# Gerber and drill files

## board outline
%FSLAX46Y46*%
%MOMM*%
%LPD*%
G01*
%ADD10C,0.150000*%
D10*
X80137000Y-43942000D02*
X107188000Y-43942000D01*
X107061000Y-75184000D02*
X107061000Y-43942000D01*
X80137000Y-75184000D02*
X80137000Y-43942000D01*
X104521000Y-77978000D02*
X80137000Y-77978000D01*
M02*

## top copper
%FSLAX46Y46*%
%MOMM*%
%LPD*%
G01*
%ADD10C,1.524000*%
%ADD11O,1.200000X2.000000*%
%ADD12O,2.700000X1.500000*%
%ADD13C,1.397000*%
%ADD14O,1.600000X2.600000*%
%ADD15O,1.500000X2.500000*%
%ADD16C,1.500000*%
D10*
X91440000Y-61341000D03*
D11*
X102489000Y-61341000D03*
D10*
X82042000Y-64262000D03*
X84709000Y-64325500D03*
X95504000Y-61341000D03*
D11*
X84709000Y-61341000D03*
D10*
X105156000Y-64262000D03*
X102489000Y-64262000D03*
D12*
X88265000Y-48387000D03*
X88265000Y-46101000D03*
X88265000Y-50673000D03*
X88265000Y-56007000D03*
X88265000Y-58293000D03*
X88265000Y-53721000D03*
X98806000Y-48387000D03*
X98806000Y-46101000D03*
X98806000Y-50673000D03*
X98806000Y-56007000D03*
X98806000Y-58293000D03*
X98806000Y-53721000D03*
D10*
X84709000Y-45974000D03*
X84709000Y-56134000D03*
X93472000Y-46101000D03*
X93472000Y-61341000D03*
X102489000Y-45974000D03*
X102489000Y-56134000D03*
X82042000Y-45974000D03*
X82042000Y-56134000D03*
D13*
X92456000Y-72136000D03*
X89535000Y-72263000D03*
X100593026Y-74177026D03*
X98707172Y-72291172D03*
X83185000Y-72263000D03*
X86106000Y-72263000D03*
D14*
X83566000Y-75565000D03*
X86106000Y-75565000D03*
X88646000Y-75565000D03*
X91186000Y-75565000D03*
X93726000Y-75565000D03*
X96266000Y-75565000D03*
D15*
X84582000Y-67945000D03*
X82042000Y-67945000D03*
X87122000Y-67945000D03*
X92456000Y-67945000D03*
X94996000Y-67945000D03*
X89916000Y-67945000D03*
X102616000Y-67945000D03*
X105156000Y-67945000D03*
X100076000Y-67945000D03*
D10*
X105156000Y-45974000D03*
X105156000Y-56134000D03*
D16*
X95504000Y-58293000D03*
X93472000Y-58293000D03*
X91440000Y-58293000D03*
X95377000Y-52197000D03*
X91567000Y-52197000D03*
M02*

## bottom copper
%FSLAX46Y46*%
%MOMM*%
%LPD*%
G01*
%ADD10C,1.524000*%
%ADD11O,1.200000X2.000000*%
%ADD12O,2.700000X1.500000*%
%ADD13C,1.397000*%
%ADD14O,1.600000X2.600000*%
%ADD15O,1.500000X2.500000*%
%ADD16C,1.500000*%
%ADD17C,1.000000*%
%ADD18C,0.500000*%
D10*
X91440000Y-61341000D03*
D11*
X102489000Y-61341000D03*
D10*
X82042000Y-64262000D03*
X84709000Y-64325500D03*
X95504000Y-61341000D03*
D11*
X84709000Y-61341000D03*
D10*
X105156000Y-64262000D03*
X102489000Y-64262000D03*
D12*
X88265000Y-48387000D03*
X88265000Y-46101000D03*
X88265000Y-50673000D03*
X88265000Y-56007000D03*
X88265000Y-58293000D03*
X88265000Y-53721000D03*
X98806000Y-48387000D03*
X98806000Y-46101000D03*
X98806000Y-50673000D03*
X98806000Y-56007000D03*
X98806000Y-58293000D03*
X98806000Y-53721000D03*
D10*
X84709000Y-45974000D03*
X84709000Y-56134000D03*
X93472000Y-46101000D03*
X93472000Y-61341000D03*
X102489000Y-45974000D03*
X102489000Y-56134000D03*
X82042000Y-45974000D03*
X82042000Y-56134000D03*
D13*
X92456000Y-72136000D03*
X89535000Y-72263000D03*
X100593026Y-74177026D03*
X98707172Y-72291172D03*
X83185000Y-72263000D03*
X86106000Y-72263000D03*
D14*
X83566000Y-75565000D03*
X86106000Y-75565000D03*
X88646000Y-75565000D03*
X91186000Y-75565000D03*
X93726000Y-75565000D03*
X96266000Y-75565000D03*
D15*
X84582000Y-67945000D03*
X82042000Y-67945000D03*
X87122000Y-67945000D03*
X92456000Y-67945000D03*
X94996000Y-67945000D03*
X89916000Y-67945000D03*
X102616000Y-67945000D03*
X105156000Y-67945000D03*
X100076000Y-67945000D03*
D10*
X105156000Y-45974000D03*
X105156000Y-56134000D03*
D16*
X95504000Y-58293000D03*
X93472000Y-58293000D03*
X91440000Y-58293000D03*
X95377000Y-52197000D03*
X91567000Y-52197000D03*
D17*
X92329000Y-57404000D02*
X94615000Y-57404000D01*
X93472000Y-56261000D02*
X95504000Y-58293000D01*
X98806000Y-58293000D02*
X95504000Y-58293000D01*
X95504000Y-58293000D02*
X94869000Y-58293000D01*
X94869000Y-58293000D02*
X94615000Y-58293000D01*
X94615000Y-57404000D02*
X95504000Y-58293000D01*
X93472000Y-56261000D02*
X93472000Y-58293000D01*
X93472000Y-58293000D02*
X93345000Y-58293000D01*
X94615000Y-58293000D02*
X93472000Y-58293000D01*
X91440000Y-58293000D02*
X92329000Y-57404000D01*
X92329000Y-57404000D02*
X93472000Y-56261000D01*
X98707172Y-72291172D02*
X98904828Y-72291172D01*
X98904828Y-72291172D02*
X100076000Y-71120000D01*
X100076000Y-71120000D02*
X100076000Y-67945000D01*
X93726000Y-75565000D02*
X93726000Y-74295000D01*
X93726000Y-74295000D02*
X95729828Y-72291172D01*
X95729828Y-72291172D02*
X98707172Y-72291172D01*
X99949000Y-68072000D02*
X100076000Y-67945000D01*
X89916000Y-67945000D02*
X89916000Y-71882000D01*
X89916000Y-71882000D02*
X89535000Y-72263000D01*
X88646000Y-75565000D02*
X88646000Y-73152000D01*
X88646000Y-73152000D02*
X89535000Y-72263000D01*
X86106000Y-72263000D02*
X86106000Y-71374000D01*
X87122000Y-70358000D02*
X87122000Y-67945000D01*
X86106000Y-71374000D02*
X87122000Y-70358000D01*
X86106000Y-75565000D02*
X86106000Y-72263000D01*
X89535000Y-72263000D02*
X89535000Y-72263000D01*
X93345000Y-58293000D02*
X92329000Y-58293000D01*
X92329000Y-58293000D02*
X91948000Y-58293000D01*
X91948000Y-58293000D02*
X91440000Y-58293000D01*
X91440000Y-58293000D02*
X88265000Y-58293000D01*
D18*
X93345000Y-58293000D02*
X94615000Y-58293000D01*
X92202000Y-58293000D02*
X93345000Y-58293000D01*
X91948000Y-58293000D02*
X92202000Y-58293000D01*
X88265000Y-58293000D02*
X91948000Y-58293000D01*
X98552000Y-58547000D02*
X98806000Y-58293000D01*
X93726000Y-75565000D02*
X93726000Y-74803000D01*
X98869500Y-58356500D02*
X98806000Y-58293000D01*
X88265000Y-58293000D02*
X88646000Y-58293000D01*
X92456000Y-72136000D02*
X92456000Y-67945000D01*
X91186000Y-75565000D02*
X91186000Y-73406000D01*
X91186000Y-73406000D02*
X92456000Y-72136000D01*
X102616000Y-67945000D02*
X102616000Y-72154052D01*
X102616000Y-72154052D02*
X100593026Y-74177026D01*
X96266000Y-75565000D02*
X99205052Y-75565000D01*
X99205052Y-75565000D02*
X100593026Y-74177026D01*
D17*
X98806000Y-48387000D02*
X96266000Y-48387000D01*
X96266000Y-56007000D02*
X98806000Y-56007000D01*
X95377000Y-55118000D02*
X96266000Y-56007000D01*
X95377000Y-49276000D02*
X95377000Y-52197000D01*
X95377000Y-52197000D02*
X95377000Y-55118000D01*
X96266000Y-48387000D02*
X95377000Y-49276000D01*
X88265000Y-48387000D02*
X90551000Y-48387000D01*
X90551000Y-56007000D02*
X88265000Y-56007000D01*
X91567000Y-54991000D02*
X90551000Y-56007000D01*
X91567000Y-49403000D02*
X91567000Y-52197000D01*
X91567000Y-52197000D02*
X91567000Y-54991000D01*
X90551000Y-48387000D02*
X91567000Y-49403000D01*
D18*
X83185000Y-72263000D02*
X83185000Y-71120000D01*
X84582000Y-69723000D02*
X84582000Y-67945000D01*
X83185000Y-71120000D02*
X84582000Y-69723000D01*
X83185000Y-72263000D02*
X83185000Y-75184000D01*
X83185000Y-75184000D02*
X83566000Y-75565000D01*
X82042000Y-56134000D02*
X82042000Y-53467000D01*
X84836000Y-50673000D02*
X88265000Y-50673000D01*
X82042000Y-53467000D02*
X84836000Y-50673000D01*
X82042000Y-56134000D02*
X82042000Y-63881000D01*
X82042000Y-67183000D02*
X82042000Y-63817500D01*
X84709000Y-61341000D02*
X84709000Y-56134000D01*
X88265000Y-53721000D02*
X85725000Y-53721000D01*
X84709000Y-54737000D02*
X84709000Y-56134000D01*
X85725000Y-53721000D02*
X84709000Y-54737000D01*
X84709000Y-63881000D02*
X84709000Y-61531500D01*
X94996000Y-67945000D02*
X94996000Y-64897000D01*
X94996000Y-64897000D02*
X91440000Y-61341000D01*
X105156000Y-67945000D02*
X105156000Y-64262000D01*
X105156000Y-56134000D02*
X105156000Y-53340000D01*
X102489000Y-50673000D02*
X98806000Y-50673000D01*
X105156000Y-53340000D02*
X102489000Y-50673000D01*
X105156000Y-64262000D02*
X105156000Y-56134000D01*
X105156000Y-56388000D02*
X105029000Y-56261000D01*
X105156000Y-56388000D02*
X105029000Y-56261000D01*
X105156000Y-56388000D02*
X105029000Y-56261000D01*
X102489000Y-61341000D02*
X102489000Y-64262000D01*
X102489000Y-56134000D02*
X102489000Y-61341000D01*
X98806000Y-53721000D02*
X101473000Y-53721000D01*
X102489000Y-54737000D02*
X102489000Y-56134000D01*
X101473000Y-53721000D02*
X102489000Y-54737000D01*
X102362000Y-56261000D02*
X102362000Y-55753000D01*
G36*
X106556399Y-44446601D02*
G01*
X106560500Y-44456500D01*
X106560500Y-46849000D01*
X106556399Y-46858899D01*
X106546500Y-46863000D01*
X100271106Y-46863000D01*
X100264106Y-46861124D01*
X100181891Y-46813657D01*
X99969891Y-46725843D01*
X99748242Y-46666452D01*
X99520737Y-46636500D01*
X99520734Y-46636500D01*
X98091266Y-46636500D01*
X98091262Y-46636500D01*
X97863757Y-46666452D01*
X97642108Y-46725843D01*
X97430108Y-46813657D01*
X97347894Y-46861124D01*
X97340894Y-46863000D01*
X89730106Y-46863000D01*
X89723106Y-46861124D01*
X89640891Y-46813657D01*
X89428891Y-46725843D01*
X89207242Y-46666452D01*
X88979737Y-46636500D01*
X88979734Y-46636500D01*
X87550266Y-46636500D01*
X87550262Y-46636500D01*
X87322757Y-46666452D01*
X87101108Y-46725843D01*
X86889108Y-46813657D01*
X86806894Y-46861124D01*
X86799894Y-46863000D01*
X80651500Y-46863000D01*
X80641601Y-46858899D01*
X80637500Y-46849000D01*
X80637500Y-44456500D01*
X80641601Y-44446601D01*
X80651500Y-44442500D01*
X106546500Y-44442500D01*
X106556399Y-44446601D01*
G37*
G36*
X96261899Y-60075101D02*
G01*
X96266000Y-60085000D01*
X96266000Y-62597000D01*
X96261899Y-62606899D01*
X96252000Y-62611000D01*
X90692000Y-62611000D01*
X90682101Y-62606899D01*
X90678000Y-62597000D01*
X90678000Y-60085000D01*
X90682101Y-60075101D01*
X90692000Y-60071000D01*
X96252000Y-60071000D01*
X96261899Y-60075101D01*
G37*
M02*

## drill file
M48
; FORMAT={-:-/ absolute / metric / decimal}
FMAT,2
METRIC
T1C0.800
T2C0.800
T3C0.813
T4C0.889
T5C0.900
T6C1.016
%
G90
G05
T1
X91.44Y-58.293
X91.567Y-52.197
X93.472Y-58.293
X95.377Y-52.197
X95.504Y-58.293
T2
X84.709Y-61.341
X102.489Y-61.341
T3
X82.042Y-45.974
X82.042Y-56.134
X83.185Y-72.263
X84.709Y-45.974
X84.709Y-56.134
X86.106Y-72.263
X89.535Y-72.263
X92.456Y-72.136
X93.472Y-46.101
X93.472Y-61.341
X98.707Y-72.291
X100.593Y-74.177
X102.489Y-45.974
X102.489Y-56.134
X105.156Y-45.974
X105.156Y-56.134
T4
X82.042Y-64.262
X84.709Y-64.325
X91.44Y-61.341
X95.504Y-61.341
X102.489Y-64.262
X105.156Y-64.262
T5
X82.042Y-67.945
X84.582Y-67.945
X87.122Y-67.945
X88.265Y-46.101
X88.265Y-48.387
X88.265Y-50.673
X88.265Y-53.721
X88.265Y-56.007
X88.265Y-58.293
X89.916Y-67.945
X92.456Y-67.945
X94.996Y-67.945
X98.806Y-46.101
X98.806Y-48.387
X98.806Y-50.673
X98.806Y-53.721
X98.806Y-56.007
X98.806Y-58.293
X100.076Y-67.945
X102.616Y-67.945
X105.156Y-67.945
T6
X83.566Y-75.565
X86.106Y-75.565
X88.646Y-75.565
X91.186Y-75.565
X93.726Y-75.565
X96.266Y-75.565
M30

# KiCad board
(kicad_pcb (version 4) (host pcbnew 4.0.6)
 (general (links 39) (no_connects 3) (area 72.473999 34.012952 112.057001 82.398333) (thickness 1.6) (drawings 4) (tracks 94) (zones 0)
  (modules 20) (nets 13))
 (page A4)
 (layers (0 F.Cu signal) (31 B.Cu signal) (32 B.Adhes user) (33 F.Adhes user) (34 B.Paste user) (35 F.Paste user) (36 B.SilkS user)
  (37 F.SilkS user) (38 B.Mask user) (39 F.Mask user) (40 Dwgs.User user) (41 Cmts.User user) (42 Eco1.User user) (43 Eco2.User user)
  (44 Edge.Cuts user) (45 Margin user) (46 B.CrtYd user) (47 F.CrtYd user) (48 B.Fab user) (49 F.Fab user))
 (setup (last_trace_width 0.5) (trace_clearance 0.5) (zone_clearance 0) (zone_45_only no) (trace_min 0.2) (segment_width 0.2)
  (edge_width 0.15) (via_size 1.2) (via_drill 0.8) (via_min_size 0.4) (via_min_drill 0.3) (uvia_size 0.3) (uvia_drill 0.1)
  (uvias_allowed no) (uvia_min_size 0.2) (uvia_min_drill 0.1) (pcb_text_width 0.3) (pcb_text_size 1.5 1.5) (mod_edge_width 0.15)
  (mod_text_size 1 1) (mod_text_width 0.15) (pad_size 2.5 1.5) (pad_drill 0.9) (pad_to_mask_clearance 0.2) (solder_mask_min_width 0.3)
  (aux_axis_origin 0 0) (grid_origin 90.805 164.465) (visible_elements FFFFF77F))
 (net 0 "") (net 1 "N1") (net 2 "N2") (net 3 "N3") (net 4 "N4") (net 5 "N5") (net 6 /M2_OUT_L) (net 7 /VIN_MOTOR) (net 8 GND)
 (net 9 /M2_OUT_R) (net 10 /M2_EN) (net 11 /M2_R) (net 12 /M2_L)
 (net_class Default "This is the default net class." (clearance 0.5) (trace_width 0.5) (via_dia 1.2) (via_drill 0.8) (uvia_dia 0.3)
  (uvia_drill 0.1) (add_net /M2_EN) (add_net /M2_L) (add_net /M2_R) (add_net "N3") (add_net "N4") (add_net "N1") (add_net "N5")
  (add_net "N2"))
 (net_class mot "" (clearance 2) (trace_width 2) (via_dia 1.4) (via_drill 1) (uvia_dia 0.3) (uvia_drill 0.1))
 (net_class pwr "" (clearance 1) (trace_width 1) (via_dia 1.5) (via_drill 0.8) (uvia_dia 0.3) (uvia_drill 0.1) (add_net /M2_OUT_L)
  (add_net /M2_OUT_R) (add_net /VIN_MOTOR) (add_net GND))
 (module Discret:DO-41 (layer F.Cu) (at 97.409 61.341 180)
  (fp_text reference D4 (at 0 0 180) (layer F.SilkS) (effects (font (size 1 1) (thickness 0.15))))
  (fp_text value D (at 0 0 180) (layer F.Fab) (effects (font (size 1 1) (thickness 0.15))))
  (pad 1 thru_hole circle (at 5.969 0 180) (size 1.524 1.524) (drill 0.889) (layers *.Cu *.Mask F.SilkS) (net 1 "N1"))
  (pad 2 thru_hole oval (at -5.08 0) (size 1.2 2) (drill 0.8) (layers *.Cu *.Mask B.SilkS) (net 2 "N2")))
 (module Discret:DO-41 (layer F.Cu) (at 79.629 64.262 180)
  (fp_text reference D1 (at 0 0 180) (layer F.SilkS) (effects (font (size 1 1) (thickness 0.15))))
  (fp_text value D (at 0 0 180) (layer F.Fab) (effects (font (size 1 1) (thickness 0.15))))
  (pad 1 thru_hole circle (at -2.413 0 180) (size 1.524 1.524) (drill 0.889) (layers *.Cu *.Mask F.SilkS) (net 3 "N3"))
  (pad 2 thru_hole circle (at -5.08 -0.0635 180) (size 1.524 1.524) (drill 0.889) (layers *.Cu *.Mask F.SilkS) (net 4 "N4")))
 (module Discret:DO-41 (layer F.Cu) (at 89.789 61.341)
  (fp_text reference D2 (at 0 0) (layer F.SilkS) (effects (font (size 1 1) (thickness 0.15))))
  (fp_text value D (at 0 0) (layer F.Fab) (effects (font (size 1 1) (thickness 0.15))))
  (pad 1 thru_hole circle (at 5.715 0) (size 1.524 1.524) (drill 0.889) (layers *.Cu *.Mask F.SilkS) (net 1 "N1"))
  (pad 2 thru_hole oval (at -5.08 0 180) (size 1.2 2) (drill 0.8) (layers *.Cu *.Mask B.SilkS) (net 4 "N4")))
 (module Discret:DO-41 (layer F.Cu) (at 104.902 64.262)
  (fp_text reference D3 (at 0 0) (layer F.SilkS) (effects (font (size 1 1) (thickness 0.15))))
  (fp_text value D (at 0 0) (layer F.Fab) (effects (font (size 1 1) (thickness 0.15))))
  (pad 1 thru_hole circle (at 0.254 0) (size 1.524 1.524) (drill 0.889) (layers *.Cu *.Mask F.SilkS) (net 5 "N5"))
  (pad 2 thru_hole circle (at -2.413 0) (size 1.524 1.524) (drill 0.889) (layers *.Cu *.Mask F.SilkS) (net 2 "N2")))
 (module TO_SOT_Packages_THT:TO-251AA (layer F.Cu) (at 88.265 50.673 90)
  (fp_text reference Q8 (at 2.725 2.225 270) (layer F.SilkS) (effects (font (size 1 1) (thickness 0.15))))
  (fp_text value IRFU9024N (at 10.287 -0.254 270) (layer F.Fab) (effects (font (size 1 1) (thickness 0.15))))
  (pad 2 thru_hole oval (at 2.286 0 270) (size 1.5 2.7) (drill 0.9) (layers *.Cu *.Mask F.SilkS) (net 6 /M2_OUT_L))
  (pad 3 thru_hole oval (at 4.572 0 270) (size 1.5 2.7) (drill 0.9) (layers *.Cu *.Mask F.SilkS) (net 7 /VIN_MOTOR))
  (pad 1 thru_hole oval (at 0 0 270) (size 1.5 2.7) (drill 0.9) (layers *.Cu *.Mask F.SilkS) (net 3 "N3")))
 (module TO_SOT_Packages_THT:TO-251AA (layer F.Cu) (at 88.265 53.721 270)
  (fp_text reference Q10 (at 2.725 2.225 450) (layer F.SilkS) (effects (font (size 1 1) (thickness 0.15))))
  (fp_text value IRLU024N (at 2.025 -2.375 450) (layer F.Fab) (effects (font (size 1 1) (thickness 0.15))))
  (pad 2 thru_hole oval (at 2.286 0 90) (size 1.5 2.7) (drill 0.9) (layers *.Cu *.Mask F.SilkS) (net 6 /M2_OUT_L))
  (pad 3 thru_hole oval (at 4.572 0 90) (size 1.5 2.7) (drill 0.9) (layers *.Cu *.Mask F.SilkS) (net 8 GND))
  (pad 1 thru_hole oval (at 0 0 90) (size 1.5 2.7) (drill 0.9) (layers *.Cu *.Mask F.SilkS) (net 4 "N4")))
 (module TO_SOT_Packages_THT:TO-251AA (layer F.Cu) (at 98.806 50.673 90)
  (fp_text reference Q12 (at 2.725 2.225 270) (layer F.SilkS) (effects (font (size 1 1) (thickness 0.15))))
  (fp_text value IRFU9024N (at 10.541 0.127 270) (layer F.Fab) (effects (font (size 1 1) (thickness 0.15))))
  (pad 2 thru_hole oval (at 2.286 0 270) (size 1.5 2.7) (drill 0.9) (layers *.Cu *.Mask F.SilkS) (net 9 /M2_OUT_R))
  (pad 3 thru_hole oval (at 4.572 0 270) (size 1.5 2.7) (drill 0.9) (layers *.Cu *.Mask F.SilkS) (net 7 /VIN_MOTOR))
  (pad 1 thru_hole oval (at 0 0 270) (size 1.5 2.7) (drill 0.9) (layers *.Cu *.Mask F.SilkS) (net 5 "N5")))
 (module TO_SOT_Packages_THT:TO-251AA (layer F.Cu) (at 98.806 53.721 270)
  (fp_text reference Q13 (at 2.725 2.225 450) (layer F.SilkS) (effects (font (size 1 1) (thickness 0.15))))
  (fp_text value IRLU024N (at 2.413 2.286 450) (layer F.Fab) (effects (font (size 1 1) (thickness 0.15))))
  (pad 2 thru_hole oval (at 2.286 0 90) (size 1.5 2.7) (drill 0.9) (layers *.Cu *.Mask F.SilkS) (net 9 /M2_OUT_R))
  (pad 3 thru_hole oval (at 4.572 0 90) (size 1.5 2.7) (drill 0.9) (layers *.Cu *.Mask F.SilkS) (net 8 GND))
  (pad 1 thru_hole oval (at 0 0 90) (size 1.5 2.7) (drill 0.9) (layers *.Cu *.Mask F.SilkS) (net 2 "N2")))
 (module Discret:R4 (layer F.Cu) (at 84.709 51.054 270)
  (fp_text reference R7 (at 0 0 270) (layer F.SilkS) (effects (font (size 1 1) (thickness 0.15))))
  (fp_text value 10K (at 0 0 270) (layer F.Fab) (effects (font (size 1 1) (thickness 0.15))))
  (pad 1 thru_hole circle (at -5.08 0 270) (size 1.524 1.524) (drill 0.8128) (layers *.Cu *.Mask F.SilkS) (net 7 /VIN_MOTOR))
  (pad 2 thru_hole circle (at 5.08 0 270) (size 1.524 1.524) (drill 0.8128) (layers *.Cu *.Mask F.SilkS) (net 4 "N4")))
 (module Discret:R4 (layer F.Cu) (at 93.472 51.308 270)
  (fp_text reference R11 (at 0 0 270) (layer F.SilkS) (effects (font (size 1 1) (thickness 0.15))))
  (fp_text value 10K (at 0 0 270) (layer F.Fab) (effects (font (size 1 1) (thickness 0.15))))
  (pad 1 thru_hole circle (at -5.207 0 270) (size 1.524 1.524) (drill 0.8128) (layers *.Cu *.Mask F.SilkS) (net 7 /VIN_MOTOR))
  (pad 2 thru_hole circle (at 10.033 0 270) (size 1.524 1.524) (drill 0.8128) (layers *.Cu *.Mask F.SilkS) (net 1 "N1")))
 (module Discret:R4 (layer F.Cu) (at 102.489 51.054 270)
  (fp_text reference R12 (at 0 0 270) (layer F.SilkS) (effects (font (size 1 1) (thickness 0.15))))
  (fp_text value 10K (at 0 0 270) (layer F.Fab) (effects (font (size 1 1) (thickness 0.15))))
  (pad 1 thru_hole circle (at -5.08 0 270) (size 1.524 1.524) (drill 0.8128) (layers *.Cu *.Mask F.SilkS) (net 7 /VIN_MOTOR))
  (pad 2 thru_hole circle (at 5.08 0 270) (size 1.524 1.524) (drill 0.8128) (layers *.Cu *.Mask F.SilkS) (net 2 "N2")))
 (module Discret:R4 (layer F.Cu) (at 82.042 51.054 270)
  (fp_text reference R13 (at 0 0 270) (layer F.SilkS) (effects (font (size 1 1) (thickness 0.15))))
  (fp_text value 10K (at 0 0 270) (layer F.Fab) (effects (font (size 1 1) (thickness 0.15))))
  (pad 1 thru_hole circle (at -5.08 0 270) (size 1.524 1.524) (drill 0.8128) (layers *.Cu *.Mask F.SilkS) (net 7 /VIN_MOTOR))
  (pad 2 thru_hole circle (at 5.08 0 270) (size 1.524 1.524) (drill 0.8128) (layers *.Cu *.Mask F.SilkS) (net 3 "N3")))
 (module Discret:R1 (layer F.Cu) (at 91.186 72.136 180)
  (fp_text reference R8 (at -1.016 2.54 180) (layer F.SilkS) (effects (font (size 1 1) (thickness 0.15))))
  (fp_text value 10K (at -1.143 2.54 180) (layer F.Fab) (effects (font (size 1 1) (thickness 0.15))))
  (pad 1 thru_hole circle (at -1.27 0 180) (size 1.397 1.397) (drill 0.8128) (layers *.Cu *.Mask F.SilkS) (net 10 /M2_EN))
  (pad 2 thru_hole circle (at 1.651 -0.127 180) (size 1.397 1.397) (drill 0.8128) (layers *.Cu *.Mask F.SilkS) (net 8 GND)))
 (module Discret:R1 (layer F.Cu) (at 99.695 73.279 135)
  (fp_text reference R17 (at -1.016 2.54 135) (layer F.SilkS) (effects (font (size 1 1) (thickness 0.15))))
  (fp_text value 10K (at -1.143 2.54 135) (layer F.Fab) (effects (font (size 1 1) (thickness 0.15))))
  (pad 1 thru_hole circle (at -1.27 0 135) (size 1.397 1.397) (drill 0.8128) (layers *.Cu *.Mask F.SilkS) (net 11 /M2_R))
  (pad 2 thru_hole circle (at 1.397 0 135) (size 1.397 1.397) (drill 0.8128) (layers *.Cu *.Mask F.SilkS) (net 8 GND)))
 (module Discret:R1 (layer F.Cu) (at 84.836 72.263)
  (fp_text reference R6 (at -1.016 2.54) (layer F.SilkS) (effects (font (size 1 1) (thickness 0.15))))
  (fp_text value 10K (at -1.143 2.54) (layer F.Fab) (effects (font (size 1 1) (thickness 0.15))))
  (pad 1 thru_hole circle (at -1.651 0) (size 1.397 1.397) (drill 0.8128) (layers *.Cu *.Mask F.SilkS) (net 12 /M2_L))
  (pad 2 thru_hole circle (at 1.27 0) (size 1.397 1.397) (drill 0.8128) (layers *.Cu *.Mask F.SilkS) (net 8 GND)))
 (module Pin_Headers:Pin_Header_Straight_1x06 (layer F.Cu) (at 83.566 75.565 90)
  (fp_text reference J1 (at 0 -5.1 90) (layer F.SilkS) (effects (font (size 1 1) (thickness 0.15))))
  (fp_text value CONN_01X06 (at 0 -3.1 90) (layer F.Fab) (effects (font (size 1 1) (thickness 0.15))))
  (pad 1 thru_hole oval (at 0 0 90) (size 2.6 1.6) (drill 1.016) (layers *.Cu *.Mask F.SilkS) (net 12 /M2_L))
  (pad 2 thru_hole oval (at 0 2.54 90) (size 2.6 1.6) (drill 1.016) (layers *.Cu *.Mask F.SilkS) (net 8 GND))
  (pad 3 thru_hole oval (at 0 5.08 90) (size 2.6 1.6) (drill 1.016) (layers *.Cu *.Mask F.SilkS) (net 8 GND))
  (pad 4 thru_hole oval (at 0 7.62 90) (size 2.6 1.6) (drill 1.016) (layers *.Cu *.Mask F.SilkS) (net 10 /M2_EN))
  (pad 5 thru_hole oval (at 0 10.16 90) (size 2.6 1.6) (drill 1.016) (layers *.Cu *.Mask F.SilkS) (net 8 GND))
  (pad 6 thru_hole oval (at 0 12.7 90) (size 2.6 1.6) (drill 1.016) (layers *.Cu *.Mask F.SilkS) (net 11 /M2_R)))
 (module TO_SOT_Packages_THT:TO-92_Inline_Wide (layer F.Cu) (at 87.122 67.945 180)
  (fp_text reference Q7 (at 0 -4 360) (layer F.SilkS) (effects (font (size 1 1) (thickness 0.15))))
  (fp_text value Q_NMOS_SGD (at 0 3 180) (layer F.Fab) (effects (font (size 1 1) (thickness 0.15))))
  (pad 2 thru_hole oval (at 2.54 0 270) (size 2.5 1.5) (drill 0.9) (layers *.Cu *.Mask F.SilkS) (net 12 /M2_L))
  (pad 3 thru_hole oval (at 5.08 0 270) (size 2.5 1.5) (drill 0.9) (layers *.Cu *.Mask F.SilkS) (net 3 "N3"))
  (pad 1 thru_hole oval (at 0 0 270) (size 2.5 1.5) (drill 0.9) (layers *.Cu *.Mask F.SilkS) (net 8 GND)))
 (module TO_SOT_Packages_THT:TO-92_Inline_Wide (layer F.Cu) (at 89.916 67.945)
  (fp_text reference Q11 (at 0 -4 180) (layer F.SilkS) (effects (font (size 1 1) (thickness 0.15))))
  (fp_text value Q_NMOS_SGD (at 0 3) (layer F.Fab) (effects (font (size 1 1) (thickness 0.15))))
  (pad 2 thru_hole oval (at 2.54 0 90) (size 2.5 1.5) (drill 0.9) (layers *.Cu *.Mask F.SilkS) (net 10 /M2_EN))
  (pad 3 thru_hole oval (at 5.08 0 90) (size 2.5 1.5) (drill 0.9) (layers *.Cu *.Mask F.SilkS) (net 1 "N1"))
  (pad 1 thru_hole oval (at 0 0 90) (size 2.5 1.5) (drill 0.9) (layers *.Cu *.Mask F.SilkS) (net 8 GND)))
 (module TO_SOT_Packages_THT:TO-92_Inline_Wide (layer F.Cu) (at 100.076 67.945)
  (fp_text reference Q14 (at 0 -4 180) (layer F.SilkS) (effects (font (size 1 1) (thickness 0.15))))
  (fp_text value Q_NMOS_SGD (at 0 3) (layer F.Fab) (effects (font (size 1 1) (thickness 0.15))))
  (pad 2 thru_hole oval (at 2.54 0 90) (size 2.5 1.5) (drill 0.9) (layers *.Cu *.Mask F.SilkS) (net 11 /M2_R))
  (pad 3 thru_hole oval (at 5.08 0 90) (size 2.5 1.5) (drill 0.9) (layers *.Cu *.Mask F.SilkS) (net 5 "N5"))
  (pad 1 thru_hole oval (at 0 0 90) (size 2.5 1.5) (drill 0.9) (layers *.Cu *.Mask F.SilkS) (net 8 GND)))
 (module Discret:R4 (layer F.Cu) (at 105.156 51.054 270)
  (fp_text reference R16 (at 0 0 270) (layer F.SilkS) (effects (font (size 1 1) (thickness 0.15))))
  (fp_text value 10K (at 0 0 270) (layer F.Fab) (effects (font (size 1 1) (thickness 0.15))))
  (pad 1 thru_hole circle (at -5.08 0 270) (size 1.524 1.524) (drill 0.8128) (layers *.Cu *.Mask F.SilkS) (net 7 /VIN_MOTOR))
  (pad 2 thru_hole circle (at 5.08 0 270) (size 1.524 1.524) (drill 0.8128) (layers *.Cu *.Mask F.SilkS) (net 5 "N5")))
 (gr_line (start 80.137 43.942) (end 107.188 43.942) (angle 90) (layer Edge.Cuts) (width 0.15))
 (gr_line (start 107.061 75.184) (end 107.061 43.942) (angle 90) (layer Edge.Cuts) (width 0.15))
 (gr_line (start 80.137 75.184) (end 80.137 43.942) (angle 90) (layer Edge.Cuts) (width 0.15))
 (gr_line (start 104.521 77.978) (end 80.137 77.978) (angle 90) (layer Edge.Cuts) (width 0.15))
 (segment (start 92.329 57.404) (end 94.615 57.404) (width 1) (layer B.Cu) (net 8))
 (via (at 95.504 58.293) (size 1.5) (drill 0.8) (layers F.Cu B.Cu) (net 8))
 (segment (start 93.472 56.261) (end 95.504 58.293) (width 1) (layer B.Cu) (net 8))
 (segment (start 98.806 58.293) (end 95.504 58.293) (width 1) (layer B.Cu) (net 8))
 (segment (start 95.504 58.293) (end 94.869 58.293) (width 1) (layer B.Cu) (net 8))
 (segment (start 94.869 58.293) (end 94.615 58.293) (width 1) (layer B.Cu) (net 8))
 (segment (start 94.615 57.404) (end 95.504 58.293) (width 1) (layer B.Cu) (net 8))
 (segment (start 93.472 56.261) (end 93.472 58.293) (width 1) (layer B.Cu) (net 8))
 (via (at 93.472 58.293) (size 1.5) (drill 0.8) (layers F.Cu B.Cu) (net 8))
 (segment (start 93.472 58.293) (end 93.345 58.293) (width 1) (layer B.Cu) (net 8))
 (segment (start 94.615 58.293) (end 93.472 58.293) (width 1) (layer B.Cu) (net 8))
 (segment (start 91.44 58.293) (end 92.329 57.404) (width 1) (layer B.Cu) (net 8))
 (segment (start 92.329 57.404) (end 93.472 56.261) (width 1) (layer B.Cu) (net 8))
 (via (at 91.44 58.293) (size 1.5) (drill 0.8) (layers F.Cu B.Cu) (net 8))
 (segment (start 98.707172 72.291172) (end 98.904828 72.291172) (width 1) (layer B.Cu) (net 8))
 (segment (start 98.904828 72.291172) (end 100.076 71.12) (width 1) (layer B.Cu) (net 8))
 (segment (start 100.076 71.12) (end 100.076 67.945) (width 1) (layer B.Cu) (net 8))
 (segment (start 93.726 75.565) (end 93.726 74.295) (width 1) (layer B.Cu) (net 8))
 (segment (start 93.726 74.295) (end 95.729828 72.291172) (width 1) (layer B.Cu) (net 8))
 (segment (start 95.729828 72.291172) (end 98.707172 72.291172) (width 1) (layer B.Cu) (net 8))
 (segment (start 99.949 68.072) (end 100.076 67.945) (width 1) (layer B.Cu) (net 8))
 (segment (start 89.916 67.945) (end 89.916 71.882) (width 1) (layer B.Cu) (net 8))
 (segment (start 89.916 71.882) (end 89.535 72.263) (width 1) (layer B.Cu) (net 8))
 (segment (start 88.646 75.565) (end 88.646 73.152) (width 1) (layer B.Cu) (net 8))
 (segment (start 88.646 73.152) (end 89.535 72.263) (width 1) (layer B.Cu) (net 8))
 (segment (start 86.106 72.263) (end 86.106 71.374) (width 1) (layer B.Cu) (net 8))
 (segment (start 87.122 70.358) (end 87.122 67.945) (width 1) (layer B.Cu) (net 8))
 (segment (start 86.106 71.374) (end 87.122 70.358) (width 1) (layer B.Cu) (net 8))
 (segment (start 86.106 75.565) (end 86.106 72.263) (width 1) (layer B.Cu) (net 8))
 (segment (start 89.535 72.263) (end 89.535 72.263) (width 1) (layer B.Cu) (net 8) (status 30))
 (segment (start 93.345 58.293) (end 92.329 58.293) (width 1) (layer B.Cu) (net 8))
 (segment (start 92.329 58.293) (end 91.948 58.293) (width 1) (layer B.Cu) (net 8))
 (segment (start 91.948 58.293) (end 91.44 58.293) (width 1) (layer B.Cu) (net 8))
 (segment (start 91.44 58.293) (end 88.265 58.293) (width 1) (layer B.Cu) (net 8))
 (segment (start 93.345 58.293) (end 94.615 58.293) (width 0.5) (layer B.Cu) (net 8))
 (segment (start 92.202 58.293) (end 93.345 58.293) (width 0.5) (layer B.Cu) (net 8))
 (segment (start 91.948 58.293) (end 92.202 58.293) (width 0.5) (layer B.Cu) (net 8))
 (segment (start 88.265 58.293) (end 91.948 58.293) (width 0.5) (layer B.Cu) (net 8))
 (segment (start 98.552 58.547) (end 98.806 58.293) (width 0.5) (layer B.Cu) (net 8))
 (segment (start 93.726 75.565) (end 93.726 74.803) (width 0.5) (layer B.Cu) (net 8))
 (segment (start 98.8695 58.3565) (end 98.806 58.293) (width 0.5) (layer B.Cu) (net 8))
 (segment (start 88.265 58.293) (end 88.646 58.293) (width 0.5) (layer B.Cu) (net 8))
 (segment (start 92.456 72.136) (end 92.456 67.945) (width 0.5) (layer B.Cu) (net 10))
 (segment (start 91.186 75.565) (end 91.186 73.406) (width 0.5) (layer B.Cu) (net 10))
 (segment (start 91.186 73.406) (end 92.456 72.136) (width 0.5) (layer B.Cu) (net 10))
 (segment (start 102.616 67.945) (end 102.616 72.154052) (width 0.5) (layer B.Cu) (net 11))
 (segment (start 102.616 72.154052) (end 100.593026 74.177026) (width 0.5) (layer B.Cu) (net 11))
 (segment (start 96.266 75.565) (end 99.205052 75.565) (width 0.5) (layer B.Cu) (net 11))
 (segment (start 99.205052 75.565) (end 100.593026 74.177026) (width 0.5) (layer B.Cu) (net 11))
 (via (at 95.377 52.197) (size 1.5) (drill 0.8) (layers F.Cu B.Cu) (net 9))
 (segment (start 98.806 48.387) (end 96.266 48.387) (width 1) (layer B.Cu) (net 9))
 (segment (start 96.266 56.007) (end 98.806 56.007) (width 1) (layer B.Cu) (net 9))
 (segment (start 95.377 55.118) (end 96.266 56.007) (width 1) (layer B.Cu) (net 9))
 (segment (start 95.377 49.276) (end 95.377 52.197) (width 1) (layer B.Cu) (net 9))
 (segment (start 95.377 52.197) (end 95.377 55.118) (width 1) (layer B.Cu) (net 9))
 (segment (start 96.266 48.387) (end 95.377 49.276) (width 1) (layer B.Cu) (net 9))
 (via (at 91.567 52.197) (size 1.5) (drill 0.8) (layers F.Cu B.Cu) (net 6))
 (segment (start 88.265 48.387) (end 90.551 48.387) (width 1) (layer B.Cu) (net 6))
 (segment (start 90.551 56.007) (end 88.265 56.007) (width 1) (layer B.Cu) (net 6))
 (segment (start 91.567 54.991) (end 90.551 56.007) (width 1) (layer B.Cu) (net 6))
 (segment (start 91.567 49.403) (end 91.567 52.197) (width 1) (layer B.Cu) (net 6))
 (segment (start 91.567 52.197) (end 91.567 54.991) (width 1) (layer B.Cu) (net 6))
 (segment (start 90.551 48.387) (end 91.567 49.403) (width 1) (layer B.Cu) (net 6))
 (segment (start 83.185 72.263) (end 83.185 71.12) (width 0.5) (layer B.Cu) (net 12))
 (segment (start 84.582 69.723) (end 84.582 67.945) (width 0.5) (layer B.Cu) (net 12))
 (segment (start 83.185 71.12) (end 84.582 69.723) (width 0.5) (layer B.Cu) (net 12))
 (segment (start 83.185 72.263) (end 83.185 75.184) (width 0.5) (layer B.Cu) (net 12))
 (segment (start 83.185 75.184) (end 83.566 75.565) (width 0.5) (layer B.Cu) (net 12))
 (segment (start 82.042 56.134) (end 82.042 53.467) (width 0.5) (layer B.Cu) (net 3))
 (segment (start 84.836 50.673) (end 88.265 50.673) (width 0.5) (layer B.Cu) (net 3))
 (segment (start 82.042 53.467) (end 84.836 50.673) (width 0.5) (layer B.Cu) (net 3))
 (segment (start 82.042 56.134) (end 82.042 63.881) (width 0.5) (layer B.Cu) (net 3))
 (segment (start 82.042 67.183) (end 82.042 63.8175) (width 0.5) (layer B.Cu) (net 3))
 (segment (start 84.709 61.341) (end 84.709 56.134) (width 0.5) (layer B.Cu) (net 4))
 (segment (start 88.265 53.721) (end 85.725 53.721) (width 0.5) (layer B.Cu) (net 4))
 (segment (start 84.709 54.737) (end 84.709 56.134) (width 0.5) (layer B.Cu) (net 4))
 (segment (start 85.725 53.721) (end 84.709 54.737) (width 0.5) (layer B.Cu) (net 4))
 (segment (start 84.709 63.881) (end 84.709 61.5315) (width 0.5) (layer B.Cu) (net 4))
 (segment (start 94.996 67.945) (end 94.996 64.897) (width 0.5) (layer B.Cu) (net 1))
 (segment (start 94.996 64.897) (end 91.44 61.341) (width 0.5) (layer B.Cu) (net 1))
 (segment (start 105.156 67.945) (end 105.156 64.262) (width 0.5) (layer B.Cu) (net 5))
 (segment (start 105.156 56.134) (end 105.156 53.34) (width 0.5) (layer B.Cu) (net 5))
 (segment (start 102.489 50.673) (end 98.806 50.673) (width 0.5) (layer B.Cu) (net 5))
 (segment (start 105.156 53.34) (end 102.489 50.673) (width 0.5) (layer B.Cu) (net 5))
 (segment (start 105.156 64.262) (end 105.156 56.134) (width 0.5) (layer B.Cu) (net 5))
 (segment (start 105.156 56.388) (end 105.029 56.261) (width 0.5) (layer B.Cu) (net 5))
 (segment (start 105.156 56.388) (end 105.029 56.261) (width 0.5) (layer B.Cu) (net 5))
 (segment (start 105.156 56.388) (end 105.029 56.261) (width 0.5) (layer B.Cu) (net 5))
 (segment (start 102.489 61.341) (end 102.489 64.262) (width 0.5) (layer B.Cu) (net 2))
 (segment (start 102.489 56.134) (end 102.489 61.341) (width 0.5) (layer B.Cu) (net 2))
 (segment (start 98.806 53.721) (end 101.473 53.721) (width 0.5) (layer B.Cu) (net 2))
 (segment (start 102.489 54.737) (end 102.489 56.134) (width 0.5) (layer B.Cu) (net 2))
 (segment (start 101.473 53.721) (end 102.489 54.737) (width 0.5) (layer B.Cu) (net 2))
 (segment (start 102.362 56.261) (end 102.362 55.753) (width 0.5) (layer B.Cu) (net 2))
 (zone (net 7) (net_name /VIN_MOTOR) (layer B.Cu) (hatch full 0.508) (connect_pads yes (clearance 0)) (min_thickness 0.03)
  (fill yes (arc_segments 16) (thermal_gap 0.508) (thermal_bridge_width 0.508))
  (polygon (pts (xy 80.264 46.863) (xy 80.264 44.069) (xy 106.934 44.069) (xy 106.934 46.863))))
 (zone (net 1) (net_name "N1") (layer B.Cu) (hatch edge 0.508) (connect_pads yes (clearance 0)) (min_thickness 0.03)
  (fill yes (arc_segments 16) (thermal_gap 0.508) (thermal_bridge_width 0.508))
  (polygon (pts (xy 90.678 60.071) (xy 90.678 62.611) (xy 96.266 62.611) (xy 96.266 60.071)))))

